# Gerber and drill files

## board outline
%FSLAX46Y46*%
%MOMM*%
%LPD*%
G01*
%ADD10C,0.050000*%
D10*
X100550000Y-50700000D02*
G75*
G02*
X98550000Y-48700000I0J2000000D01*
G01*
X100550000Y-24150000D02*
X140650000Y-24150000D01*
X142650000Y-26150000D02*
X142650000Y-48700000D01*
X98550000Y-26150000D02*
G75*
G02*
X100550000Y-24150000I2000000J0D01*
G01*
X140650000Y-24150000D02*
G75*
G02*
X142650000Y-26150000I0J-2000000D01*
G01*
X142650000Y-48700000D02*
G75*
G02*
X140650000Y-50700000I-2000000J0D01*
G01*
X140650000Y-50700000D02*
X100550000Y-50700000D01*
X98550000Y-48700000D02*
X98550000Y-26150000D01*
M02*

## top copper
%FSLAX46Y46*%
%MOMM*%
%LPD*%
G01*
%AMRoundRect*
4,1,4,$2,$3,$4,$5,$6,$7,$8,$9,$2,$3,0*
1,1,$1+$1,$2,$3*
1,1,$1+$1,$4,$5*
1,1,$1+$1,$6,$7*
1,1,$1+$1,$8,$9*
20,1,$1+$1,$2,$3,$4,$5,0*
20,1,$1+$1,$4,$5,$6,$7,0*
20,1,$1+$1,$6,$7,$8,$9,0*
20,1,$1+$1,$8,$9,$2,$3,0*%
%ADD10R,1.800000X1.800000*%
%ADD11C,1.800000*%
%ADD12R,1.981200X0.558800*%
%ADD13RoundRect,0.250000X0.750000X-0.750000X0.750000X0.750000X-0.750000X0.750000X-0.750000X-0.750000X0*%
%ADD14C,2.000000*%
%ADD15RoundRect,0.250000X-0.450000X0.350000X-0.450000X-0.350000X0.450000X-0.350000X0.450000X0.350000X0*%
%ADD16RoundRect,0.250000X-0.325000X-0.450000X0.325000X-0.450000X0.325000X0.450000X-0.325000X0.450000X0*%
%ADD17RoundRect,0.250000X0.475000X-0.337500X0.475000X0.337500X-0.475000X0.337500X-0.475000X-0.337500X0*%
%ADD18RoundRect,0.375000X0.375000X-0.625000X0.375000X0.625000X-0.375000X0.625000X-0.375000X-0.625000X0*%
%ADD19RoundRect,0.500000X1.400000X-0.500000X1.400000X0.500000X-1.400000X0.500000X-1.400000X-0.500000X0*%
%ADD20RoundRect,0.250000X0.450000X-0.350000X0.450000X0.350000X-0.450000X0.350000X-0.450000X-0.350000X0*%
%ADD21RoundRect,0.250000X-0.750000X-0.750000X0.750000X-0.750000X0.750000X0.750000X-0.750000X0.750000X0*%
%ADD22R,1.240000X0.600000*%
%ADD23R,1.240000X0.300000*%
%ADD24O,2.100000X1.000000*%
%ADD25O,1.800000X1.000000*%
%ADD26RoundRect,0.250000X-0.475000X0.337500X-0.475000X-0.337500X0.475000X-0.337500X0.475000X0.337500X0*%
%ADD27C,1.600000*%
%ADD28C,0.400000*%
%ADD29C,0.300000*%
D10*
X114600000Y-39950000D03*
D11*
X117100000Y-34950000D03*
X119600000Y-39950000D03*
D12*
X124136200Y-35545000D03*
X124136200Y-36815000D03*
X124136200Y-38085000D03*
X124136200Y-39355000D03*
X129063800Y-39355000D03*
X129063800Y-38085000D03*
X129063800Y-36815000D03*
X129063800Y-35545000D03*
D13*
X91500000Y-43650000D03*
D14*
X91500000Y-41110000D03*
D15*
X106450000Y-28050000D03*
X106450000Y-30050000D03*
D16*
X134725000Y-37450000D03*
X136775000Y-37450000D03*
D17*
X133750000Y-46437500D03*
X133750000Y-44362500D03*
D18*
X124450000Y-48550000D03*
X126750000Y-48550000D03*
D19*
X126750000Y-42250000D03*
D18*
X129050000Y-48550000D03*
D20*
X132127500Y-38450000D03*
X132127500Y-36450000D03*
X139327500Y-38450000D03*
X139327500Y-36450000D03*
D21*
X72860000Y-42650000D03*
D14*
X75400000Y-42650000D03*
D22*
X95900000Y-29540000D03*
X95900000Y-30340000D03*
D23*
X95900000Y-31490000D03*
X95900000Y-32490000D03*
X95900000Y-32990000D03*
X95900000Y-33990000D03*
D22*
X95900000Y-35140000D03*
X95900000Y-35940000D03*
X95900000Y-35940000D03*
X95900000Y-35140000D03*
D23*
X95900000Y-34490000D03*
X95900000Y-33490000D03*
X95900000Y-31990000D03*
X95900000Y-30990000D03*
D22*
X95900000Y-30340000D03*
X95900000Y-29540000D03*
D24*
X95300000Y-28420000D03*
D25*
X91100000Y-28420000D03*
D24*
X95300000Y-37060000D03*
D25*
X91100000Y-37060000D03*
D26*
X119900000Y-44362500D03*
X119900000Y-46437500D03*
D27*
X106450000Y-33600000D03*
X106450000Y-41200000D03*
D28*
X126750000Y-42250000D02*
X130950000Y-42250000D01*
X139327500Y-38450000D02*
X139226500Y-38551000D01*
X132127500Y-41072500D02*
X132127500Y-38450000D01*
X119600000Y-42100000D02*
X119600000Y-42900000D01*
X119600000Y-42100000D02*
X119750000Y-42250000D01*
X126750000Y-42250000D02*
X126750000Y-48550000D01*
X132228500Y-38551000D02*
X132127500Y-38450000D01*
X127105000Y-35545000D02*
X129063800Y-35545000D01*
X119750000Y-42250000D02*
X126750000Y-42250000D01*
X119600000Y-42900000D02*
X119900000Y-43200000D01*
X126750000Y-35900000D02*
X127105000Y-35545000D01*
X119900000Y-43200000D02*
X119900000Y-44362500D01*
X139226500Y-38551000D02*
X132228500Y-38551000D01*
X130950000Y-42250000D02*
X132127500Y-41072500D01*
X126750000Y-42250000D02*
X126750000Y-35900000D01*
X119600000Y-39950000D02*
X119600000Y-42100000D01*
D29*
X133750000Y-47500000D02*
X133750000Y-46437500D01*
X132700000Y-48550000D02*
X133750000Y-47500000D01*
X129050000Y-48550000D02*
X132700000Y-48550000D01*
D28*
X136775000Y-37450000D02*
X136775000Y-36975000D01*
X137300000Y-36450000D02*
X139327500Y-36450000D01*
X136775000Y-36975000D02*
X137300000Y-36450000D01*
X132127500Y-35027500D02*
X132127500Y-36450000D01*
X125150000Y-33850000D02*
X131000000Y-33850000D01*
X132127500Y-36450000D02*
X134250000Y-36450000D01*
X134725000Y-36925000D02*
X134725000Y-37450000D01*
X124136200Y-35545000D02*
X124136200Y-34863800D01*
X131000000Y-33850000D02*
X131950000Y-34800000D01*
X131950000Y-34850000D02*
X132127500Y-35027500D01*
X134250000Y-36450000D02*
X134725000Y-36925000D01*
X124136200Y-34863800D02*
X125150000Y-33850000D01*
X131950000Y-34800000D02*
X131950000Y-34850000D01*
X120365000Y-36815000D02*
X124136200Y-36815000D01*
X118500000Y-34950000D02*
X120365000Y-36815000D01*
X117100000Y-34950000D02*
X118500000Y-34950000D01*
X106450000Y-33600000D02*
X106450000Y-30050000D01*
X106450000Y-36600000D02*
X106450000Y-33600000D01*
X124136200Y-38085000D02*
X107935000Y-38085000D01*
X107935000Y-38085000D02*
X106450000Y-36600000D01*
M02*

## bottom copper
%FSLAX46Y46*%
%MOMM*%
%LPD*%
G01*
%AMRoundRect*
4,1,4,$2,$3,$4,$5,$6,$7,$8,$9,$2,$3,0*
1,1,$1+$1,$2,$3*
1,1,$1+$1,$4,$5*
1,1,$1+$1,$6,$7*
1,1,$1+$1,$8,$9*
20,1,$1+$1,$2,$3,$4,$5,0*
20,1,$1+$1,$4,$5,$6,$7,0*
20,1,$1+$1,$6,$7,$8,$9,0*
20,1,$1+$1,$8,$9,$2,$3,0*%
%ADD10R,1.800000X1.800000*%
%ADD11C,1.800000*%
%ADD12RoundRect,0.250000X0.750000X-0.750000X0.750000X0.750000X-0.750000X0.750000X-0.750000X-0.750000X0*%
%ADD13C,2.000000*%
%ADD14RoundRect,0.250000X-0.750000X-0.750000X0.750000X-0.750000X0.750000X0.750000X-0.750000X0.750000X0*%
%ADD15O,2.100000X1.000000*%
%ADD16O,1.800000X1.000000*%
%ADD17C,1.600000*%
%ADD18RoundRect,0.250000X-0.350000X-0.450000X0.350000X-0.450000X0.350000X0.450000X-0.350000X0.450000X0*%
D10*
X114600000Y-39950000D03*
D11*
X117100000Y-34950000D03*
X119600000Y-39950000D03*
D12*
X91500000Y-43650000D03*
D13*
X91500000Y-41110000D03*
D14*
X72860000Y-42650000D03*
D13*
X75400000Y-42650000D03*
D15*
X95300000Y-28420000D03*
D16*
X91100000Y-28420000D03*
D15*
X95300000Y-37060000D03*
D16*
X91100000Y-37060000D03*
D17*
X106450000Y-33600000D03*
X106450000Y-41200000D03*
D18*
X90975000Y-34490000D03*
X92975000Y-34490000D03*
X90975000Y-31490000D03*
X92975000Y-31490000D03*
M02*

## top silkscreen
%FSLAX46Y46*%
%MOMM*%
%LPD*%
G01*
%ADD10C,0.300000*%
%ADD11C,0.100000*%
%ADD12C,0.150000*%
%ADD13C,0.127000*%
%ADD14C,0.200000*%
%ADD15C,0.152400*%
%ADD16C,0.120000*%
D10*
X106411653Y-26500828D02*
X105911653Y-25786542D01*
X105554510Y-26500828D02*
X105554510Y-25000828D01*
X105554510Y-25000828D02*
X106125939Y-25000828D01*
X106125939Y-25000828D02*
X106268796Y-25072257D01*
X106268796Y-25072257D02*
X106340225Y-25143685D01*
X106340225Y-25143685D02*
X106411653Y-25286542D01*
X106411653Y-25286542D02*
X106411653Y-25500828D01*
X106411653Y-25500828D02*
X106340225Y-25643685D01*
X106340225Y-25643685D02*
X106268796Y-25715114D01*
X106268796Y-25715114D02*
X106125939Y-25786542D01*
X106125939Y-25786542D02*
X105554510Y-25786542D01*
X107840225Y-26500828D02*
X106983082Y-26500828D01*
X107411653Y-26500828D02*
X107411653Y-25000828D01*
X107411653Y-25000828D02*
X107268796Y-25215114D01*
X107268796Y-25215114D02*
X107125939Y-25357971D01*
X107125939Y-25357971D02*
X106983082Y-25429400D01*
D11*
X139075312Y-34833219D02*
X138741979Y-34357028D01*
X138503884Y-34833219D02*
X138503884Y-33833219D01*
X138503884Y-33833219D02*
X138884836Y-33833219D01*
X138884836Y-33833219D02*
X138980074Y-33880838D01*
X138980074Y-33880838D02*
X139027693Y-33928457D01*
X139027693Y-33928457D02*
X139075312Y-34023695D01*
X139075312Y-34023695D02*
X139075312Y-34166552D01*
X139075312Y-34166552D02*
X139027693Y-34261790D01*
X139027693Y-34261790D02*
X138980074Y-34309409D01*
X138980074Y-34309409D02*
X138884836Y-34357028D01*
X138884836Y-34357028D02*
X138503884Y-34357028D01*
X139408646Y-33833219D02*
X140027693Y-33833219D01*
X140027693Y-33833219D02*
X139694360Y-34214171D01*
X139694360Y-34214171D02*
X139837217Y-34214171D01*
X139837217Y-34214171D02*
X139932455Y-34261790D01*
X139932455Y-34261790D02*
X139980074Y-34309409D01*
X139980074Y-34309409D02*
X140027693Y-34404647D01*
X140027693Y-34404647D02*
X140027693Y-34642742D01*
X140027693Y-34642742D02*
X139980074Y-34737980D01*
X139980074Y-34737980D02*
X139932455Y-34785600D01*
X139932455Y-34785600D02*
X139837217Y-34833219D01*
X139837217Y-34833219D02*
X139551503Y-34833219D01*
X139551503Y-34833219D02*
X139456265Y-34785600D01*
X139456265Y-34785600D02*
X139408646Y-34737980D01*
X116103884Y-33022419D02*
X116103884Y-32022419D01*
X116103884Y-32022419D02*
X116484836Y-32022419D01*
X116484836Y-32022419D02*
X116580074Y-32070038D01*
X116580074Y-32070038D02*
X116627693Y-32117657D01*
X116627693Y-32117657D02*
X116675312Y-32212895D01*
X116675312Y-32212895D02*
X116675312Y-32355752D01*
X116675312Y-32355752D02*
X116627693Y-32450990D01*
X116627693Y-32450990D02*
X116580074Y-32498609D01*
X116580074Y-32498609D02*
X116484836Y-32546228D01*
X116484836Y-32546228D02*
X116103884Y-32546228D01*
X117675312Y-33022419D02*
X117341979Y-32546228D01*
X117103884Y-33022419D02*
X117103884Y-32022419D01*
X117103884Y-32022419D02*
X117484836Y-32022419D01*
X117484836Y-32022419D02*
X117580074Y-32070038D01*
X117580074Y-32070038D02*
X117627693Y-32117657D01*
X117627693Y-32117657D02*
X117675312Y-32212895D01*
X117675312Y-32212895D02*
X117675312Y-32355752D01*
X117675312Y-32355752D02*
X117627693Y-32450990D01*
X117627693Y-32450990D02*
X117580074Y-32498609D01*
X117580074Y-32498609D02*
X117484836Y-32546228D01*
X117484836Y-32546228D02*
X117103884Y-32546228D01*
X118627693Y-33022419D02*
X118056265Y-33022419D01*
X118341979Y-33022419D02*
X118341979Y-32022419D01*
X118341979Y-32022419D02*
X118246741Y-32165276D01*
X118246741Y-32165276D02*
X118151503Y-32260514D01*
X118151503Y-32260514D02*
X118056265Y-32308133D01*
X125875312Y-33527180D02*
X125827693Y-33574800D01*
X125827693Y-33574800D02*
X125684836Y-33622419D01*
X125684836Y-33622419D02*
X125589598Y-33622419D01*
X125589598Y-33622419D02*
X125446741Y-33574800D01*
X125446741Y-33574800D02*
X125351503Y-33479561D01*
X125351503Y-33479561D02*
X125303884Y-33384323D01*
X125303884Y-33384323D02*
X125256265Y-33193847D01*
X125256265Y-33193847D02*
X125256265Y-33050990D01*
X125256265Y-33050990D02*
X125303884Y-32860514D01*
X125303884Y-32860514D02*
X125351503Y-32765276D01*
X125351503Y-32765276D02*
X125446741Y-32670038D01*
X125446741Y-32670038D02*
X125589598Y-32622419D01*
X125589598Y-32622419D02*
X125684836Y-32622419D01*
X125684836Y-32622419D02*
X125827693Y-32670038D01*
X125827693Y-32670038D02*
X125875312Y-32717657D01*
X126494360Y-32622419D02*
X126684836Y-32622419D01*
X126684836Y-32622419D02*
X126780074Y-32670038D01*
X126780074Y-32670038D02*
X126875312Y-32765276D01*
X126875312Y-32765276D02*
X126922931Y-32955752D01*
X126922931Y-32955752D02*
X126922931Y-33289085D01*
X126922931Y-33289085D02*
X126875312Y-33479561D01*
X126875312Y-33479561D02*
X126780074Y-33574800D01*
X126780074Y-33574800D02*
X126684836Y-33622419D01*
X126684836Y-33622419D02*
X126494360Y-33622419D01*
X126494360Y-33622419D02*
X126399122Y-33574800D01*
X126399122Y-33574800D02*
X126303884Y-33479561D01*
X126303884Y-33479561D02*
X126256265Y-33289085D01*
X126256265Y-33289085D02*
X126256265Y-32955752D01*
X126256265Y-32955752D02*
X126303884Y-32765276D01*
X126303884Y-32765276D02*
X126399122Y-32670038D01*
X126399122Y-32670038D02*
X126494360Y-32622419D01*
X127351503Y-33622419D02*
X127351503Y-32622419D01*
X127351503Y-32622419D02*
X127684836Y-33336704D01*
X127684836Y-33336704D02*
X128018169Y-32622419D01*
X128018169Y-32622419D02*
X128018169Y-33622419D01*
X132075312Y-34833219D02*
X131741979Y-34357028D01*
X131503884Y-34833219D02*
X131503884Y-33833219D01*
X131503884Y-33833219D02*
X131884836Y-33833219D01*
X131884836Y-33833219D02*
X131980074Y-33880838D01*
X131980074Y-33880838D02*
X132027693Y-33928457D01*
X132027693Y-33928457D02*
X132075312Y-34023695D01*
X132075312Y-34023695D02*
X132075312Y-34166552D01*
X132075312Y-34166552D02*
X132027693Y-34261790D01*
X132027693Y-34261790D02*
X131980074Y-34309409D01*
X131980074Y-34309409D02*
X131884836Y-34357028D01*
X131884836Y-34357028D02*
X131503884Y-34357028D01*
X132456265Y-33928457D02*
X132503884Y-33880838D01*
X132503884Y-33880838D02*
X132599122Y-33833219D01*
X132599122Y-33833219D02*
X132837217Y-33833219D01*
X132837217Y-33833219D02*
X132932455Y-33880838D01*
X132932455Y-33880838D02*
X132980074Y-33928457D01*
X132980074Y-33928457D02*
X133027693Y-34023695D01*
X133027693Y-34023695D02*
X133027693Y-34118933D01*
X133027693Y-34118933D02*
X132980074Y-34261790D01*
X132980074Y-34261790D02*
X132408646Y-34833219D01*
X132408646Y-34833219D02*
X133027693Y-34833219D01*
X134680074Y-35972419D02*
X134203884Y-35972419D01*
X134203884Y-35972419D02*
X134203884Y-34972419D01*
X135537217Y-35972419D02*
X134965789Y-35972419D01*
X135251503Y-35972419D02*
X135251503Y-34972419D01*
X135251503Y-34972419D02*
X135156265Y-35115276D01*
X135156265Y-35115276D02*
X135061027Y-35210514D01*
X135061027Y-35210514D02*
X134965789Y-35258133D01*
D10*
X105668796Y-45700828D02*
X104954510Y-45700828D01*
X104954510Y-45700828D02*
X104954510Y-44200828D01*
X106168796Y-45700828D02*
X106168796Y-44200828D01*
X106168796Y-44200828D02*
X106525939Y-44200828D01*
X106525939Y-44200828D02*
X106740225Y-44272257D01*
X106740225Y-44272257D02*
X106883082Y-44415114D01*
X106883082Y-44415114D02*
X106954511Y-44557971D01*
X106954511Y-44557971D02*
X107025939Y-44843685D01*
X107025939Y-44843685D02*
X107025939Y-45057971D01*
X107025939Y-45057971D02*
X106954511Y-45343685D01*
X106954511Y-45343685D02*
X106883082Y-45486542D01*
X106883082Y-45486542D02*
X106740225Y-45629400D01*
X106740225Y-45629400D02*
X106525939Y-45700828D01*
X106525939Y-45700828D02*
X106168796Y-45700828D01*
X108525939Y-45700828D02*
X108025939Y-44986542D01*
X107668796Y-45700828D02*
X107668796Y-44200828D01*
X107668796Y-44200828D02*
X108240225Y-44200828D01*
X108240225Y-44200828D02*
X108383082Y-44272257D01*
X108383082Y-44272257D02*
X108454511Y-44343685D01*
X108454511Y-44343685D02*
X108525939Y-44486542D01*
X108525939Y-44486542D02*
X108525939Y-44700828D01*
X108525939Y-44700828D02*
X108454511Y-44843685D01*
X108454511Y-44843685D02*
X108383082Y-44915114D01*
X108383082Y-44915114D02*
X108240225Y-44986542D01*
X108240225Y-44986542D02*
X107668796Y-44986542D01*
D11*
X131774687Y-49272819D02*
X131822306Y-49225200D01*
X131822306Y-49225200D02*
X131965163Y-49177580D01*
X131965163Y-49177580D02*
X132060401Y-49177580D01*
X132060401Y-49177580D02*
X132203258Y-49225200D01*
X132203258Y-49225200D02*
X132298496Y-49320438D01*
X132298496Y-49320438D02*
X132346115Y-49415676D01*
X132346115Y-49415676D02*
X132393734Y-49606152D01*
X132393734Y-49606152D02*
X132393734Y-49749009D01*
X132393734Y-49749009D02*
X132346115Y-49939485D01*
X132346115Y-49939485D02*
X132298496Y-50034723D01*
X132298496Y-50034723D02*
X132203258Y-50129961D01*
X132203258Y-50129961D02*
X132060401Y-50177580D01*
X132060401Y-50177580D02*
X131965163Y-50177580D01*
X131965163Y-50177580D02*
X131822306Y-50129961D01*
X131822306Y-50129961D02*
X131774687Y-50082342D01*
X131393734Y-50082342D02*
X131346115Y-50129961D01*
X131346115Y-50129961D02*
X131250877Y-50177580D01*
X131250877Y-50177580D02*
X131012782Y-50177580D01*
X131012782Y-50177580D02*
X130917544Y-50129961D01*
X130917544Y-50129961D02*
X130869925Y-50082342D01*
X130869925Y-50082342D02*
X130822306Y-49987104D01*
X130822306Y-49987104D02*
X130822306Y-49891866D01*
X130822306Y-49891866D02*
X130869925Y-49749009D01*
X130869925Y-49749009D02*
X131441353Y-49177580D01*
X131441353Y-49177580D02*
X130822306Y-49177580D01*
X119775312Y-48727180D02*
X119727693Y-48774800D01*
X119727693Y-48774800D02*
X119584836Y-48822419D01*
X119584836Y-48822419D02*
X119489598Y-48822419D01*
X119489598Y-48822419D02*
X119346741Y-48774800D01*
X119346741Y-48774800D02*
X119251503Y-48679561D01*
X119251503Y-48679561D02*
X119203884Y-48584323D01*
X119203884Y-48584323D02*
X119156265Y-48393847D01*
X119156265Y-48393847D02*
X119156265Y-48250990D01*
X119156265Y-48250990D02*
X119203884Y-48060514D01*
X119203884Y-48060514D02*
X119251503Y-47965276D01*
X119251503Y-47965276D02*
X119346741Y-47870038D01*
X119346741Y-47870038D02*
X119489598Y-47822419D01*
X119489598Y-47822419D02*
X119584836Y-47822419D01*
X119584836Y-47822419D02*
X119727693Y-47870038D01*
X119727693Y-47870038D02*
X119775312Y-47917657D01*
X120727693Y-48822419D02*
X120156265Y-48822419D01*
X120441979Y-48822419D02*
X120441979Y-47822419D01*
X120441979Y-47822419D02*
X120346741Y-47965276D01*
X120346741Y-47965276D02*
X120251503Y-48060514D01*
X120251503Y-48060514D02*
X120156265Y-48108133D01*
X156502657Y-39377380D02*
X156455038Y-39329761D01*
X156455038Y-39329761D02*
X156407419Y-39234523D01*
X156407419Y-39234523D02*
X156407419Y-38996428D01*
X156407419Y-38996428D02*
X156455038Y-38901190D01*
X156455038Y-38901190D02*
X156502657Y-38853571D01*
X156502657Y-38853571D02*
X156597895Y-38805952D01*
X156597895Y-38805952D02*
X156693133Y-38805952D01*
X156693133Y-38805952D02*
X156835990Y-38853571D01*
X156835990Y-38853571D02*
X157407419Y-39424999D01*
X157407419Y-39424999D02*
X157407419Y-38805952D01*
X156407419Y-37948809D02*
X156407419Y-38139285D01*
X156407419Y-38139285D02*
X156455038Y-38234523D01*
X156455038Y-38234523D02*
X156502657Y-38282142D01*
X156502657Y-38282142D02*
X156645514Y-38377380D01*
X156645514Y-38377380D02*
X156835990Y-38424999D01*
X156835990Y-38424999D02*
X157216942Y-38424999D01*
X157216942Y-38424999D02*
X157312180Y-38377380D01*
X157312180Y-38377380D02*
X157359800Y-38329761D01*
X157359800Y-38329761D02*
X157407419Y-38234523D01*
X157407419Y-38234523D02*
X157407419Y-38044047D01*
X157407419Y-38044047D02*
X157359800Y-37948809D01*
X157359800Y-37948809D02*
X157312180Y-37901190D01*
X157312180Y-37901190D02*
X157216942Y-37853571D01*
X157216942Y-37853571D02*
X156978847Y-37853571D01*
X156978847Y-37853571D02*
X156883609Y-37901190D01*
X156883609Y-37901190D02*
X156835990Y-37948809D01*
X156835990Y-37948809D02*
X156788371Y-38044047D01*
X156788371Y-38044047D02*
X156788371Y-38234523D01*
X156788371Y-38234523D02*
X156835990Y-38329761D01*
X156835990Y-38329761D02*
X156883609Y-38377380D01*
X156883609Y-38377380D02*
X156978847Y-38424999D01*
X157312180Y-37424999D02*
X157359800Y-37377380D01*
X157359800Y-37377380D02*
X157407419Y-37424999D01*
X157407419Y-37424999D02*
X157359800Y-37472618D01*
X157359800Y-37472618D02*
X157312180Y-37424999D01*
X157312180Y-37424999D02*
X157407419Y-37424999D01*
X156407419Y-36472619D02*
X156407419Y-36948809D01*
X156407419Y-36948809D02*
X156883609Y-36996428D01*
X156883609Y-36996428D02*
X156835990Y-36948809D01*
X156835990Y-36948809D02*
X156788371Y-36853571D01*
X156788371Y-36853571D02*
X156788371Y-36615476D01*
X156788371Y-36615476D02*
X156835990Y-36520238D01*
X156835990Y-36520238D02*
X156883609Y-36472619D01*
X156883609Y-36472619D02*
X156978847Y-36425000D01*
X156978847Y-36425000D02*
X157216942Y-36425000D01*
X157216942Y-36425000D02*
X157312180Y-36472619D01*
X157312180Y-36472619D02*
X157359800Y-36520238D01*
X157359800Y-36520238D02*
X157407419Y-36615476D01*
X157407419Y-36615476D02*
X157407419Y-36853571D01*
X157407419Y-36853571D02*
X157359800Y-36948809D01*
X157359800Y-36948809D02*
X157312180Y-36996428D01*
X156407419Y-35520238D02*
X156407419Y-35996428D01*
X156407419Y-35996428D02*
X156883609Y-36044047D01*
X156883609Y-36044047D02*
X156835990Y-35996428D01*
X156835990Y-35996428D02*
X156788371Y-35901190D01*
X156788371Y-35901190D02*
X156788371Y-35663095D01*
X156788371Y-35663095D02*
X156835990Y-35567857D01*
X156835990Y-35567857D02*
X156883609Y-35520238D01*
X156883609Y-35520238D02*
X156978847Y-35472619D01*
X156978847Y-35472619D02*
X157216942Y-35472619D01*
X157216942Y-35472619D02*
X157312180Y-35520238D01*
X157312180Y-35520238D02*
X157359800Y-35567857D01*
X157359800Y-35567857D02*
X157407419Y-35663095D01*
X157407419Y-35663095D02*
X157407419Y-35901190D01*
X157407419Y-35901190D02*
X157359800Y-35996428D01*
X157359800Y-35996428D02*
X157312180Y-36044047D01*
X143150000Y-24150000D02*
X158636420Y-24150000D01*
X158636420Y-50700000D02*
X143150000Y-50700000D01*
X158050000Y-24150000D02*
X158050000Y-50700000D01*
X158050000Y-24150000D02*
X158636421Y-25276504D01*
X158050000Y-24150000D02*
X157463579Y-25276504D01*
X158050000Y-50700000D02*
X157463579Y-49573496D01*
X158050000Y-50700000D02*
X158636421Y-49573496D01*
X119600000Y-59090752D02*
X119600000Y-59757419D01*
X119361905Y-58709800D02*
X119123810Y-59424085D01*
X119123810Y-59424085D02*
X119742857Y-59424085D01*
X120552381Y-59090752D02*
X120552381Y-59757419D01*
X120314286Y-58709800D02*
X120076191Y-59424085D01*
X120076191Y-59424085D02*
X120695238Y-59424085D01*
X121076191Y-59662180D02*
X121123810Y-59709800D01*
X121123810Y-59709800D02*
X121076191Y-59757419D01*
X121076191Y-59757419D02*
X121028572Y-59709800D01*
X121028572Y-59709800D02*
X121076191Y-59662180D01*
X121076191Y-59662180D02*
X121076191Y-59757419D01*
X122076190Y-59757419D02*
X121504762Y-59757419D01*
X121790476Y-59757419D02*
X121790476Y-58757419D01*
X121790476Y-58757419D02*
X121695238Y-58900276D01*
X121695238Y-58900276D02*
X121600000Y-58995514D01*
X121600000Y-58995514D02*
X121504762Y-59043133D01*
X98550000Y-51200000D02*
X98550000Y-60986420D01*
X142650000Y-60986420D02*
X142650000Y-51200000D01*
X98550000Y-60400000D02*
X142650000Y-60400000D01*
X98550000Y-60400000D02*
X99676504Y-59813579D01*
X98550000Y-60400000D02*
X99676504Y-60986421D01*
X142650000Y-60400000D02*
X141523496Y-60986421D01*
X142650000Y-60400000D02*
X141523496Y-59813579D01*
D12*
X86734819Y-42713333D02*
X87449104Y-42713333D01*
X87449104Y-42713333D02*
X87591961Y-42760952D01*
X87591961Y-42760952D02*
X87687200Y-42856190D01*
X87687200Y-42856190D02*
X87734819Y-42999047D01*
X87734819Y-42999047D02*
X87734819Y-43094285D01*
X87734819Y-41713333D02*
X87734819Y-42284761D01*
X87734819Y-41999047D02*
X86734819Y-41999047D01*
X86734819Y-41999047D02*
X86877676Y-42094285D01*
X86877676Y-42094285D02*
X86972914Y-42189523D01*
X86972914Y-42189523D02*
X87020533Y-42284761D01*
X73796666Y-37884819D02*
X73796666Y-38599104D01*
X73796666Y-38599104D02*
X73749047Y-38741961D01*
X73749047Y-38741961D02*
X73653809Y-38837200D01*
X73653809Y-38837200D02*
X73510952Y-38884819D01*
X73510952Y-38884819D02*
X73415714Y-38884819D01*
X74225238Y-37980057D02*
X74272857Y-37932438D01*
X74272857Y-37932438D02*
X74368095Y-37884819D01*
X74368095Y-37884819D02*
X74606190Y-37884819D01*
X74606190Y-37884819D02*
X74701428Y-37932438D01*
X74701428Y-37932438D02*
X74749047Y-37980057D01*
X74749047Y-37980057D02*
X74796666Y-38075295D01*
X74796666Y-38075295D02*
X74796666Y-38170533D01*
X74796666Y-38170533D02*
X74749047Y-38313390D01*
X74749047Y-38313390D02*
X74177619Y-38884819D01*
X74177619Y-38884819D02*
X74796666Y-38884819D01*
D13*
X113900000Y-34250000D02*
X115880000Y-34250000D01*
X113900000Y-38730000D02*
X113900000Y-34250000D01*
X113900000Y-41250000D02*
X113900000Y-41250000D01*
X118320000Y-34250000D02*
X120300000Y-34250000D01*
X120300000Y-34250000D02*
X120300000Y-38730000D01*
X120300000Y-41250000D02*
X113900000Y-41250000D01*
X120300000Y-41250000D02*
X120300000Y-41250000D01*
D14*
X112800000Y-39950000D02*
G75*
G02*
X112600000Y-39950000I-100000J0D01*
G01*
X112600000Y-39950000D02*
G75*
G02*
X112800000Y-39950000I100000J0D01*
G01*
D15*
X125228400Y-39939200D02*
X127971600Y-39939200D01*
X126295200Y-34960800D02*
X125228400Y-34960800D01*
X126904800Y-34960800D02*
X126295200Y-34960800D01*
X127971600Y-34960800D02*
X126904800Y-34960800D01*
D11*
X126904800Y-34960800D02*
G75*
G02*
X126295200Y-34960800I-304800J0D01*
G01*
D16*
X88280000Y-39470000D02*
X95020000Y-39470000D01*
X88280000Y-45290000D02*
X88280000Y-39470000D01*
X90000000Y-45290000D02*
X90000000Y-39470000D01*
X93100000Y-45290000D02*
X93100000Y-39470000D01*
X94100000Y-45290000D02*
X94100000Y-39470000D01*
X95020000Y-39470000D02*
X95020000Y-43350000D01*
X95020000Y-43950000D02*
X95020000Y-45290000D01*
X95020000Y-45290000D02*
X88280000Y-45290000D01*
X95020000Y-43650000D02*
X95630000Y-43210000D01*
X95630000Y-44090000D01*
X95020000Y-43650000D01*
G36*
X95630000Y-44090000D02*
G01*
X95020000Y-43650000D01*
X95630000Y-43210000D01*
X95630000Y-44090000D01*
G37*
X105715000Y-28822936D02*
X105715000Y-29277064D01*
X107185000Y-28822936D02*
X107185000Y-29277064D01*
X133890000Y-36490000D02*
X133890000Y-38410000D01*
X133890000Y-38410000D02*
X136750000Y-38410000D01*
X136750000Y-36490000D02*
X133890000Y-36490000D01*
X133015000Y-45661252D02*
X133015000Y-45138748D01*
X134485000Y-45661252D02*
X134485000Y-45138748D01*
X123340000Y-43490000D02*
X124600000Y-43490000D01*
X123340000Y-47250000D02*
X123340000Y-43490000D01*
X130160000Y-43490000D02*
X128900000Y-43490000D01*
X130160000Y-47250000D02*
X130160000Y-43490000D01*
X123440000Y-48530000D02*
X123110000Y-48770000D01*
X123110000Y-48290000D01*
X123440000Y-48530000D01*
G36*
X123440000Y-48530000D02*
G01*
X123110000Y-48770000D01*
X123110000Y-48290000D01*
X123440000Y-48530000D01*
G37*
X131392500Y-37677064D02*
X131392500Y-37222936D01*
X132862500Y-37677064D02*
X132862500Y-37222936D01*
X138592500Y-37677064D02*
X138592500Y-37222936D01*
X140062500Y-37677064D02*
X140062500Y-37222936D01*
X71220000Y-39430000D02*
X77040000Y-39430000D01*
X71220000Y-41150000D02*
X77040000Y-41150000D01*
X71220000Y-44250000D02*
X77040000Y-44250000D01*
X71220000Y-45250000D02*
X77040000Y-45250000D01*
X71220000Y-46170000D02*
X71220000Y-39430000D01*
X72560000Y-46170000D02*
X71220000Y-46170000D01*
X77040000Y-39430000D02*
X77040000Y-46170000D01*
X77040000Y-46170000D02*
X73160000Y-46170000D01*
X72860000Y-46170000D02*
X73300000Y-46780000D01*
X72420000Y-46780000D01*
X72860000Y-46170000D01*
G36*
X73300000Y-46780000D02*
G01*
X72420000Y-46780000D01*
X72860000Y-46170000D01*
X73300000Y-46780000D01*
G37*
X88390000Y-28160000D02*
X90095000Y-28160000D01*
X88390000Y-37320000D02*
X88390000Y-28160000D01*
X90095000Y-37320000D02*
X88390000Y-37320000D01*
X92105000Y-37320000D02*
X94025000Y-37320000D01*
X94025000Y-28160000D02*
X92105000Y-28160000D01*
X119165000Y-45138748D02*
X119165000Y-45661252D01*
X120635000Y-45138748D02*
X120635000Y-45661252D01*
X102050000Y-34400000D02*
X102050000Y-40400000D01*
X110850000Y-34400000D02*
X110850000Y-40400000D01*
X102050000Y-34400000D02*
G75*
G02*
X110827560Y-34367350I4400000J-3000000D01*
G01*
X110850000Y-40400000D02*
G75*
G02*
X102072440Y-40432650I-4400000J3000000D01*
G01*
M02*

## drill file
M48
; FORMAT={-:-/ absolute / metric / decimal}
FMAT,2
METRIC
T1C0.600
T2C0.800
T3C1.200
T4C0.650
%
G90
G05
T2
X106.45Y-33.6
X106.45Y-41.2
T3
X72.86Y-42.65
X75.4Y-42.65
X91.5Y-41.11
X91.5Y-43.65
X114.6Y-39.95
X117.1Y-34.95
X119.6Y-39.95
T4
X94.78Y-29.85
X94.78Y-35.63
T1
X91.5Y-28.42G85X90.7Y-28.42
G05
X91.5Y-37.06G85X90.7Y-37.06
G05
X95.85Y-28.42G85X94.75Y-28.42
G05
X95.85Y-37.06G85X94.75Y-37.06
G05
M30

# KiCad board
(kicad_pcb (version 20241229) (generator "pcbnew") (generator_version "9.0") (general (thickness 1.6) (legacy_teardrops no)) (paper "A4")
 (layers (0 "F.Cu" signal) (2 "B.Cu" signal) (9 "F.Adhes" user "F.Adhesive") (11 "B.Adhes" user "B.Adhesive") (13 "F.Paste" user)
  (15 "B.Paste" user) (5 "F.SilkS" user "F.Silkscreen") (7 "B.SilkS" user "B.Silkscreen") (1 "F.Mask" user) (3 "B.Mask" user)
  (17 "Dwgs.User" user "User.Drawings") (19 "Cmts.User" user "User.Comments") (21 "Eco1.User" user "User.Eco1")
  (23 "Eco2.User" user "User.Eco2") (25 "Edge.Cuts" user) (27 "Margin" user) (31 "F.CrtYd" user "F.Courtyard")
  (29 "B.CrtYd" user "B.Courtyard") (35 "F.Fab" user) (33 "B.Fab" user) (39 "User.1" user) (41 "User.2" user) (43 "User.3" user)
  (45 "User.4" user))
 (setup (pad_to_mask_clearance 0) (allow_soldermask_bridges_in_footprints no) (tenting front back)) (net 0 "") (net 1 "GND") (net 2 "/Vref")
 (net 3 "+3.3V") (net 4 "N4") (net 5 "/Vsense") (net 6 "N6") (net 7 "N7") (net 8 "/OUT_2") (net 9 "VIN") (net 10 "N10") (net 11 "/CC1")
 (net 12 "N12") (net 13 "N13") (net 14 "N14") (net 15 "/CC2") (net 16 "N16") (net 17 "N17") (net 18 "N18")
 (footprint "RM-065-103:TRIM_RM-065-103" (layer "F.Cu") (at 117.1 37.45)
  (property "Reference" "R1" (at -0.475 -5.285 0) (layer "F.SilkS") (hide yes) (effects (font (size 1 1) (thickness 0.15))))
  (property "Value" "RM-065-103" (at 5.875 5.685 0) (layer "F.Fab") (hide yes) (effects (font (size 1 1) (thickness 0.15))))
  (fp_line (start -3.2 -3.2) (end -1.22 -3.2) (stroke (width 0.127) (type solid)) (layer "F.SilkS"))
  (fp_line (start -3.2 1.28) (end -3.2 -3.2) (stroke (width 0.127) (type solid)) (layer "F.SilkS"))
  (fp_line (start -3.2 3.8) (end -3.2 3.8) (stroke (width 0.127) (type solid)) (layer "F.SilkS"))
  (fp_line (start 1.22 -3.2) (end 3.2 -3.2) (stroke (width 0.127) (type solid)) (layer "F.SilkS"))
  (fp_line (start 3.2 -3.2) (end 3.2 1.28) (stroke (width 0.127) (type solid)) (layer "F.SilkS"))
  (fp_line (start 3.2 3.8) (end -3.2 3.8) (stroke (width 0.127) (type solid)) (layer "F.SilkS"))
  (fp_line (start 3.2 3.8) (end 3.2 3.8) (stroke (width 0.127) (type solid)) (layer "F.SilkS"))
  (fp_circle (center -4.4 2.5) (end -4.3 2.5) (stroke (width 0.2) (type solid)) (fill no) (layer "F.SilkS"))
  (pad "1" thru_hole rect (at -2.5 2.5) (size 1.8 1.8) (drill 1.2) (layers "*.Cu" "*.Mask") (remove_unused_layers no) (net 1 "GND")
   (solder_mask_margin 0.102))
  (pad "2" thru_hole circle (at 0 -2.5) (size 1.8 1.8) (drill 1.2) (layers "*.Cu" "*.Mask") (remove_unused_layers no) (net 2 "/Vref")
   (solder_mask_margin 0.102))
  (pad "3" thru_hole circle (at 2.5 2.5) (size 1.8 1.8) (drill 1.2) (layers "*.Cu" "*.Mask") (remove_unused_layers no) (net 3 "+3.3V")
   (solder_mask_margin 0.102)))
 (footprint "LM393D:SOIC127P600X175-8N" (layer "F.Cu") (at 126.6 37.45)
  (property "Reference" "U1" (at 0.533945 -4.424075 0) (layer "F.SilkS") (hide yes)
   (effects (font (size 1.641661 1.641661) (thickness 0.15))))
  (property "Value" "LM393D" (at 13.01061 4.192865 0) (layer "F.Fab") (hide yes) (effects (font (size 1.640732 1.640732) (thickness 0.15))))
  (fp_line (start -1.3716 2.4892) (end 1.3716 2.4892) (stroke (width 0.1524) (type solid)) (layer "F.SilkS"))
  (fp_line (start -0.3048 -2.4892) (end -1.3716 -2.4892) (stroke (width 0.1524) (type solid)) (layer "F.SilkS"))
  (fp_line (start 0.3048 -2.4892) (end -0.3048 -2.4892) (stroke (width 0.1524) (type solid)) (layer "F.SilkS"))
  (fp_line (start 1.3716 -2.4892) (end 0.3048 -2.4892) (stroke (width 0.1524) (type solid)) (layer "F.SilkS"))
  (fp_arc (start 0.3048 -2.4892) (mid 0 -2.1844) (end -0.3048 -2.4892) (stroke (width 0.1) (type solid)) (layer "F.SilkS"))
  (pad "1" smd rect (at -2.4638 -1.905) (size 1.9812 0.5588) (layers "F.Cu" "F.Mask" "F.Paste") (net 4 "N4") (solder_mask_margin 0.102))
  (pad "2" smd rect (at -2.4638 -0.635) (size 1.9812 0.5588) (layers "F.Cu" "F.Mask" "F.Paste") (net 2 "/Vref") (solder_mask_margin 0.102))
  (pad "3" smd rect (at -2.4638 0.635) (size 1.9812 0.5588) (layers "F.Cu" "F.Mask" "F.Paste") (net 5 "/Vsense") (solder_mask_margin 0.102))
  (pad "4" smd rect (at -2.4638 1.905) (size 1.9812 0.5588) (layers "F.Cu" "F.Mask" "F.Paste") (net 1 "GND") (solder_mask_margin 0.102))
  (pad "5" smd rect (at 2.4638 1.905) (size 1.9812 0.5588) (layers "F.Cu" "F.Mask" "F.Paste") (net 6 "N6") (solder_mask_margin 0.102))
  (pad "6" smd rect (at 2.4638 0.635) (size 1.9812 0.5588) (layers "F.Cu" "F.Mask" "F.Paste") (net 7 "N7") (solder_mask_margin 0.102))
  (pad "7" smd rect (at 2.4638 -0.635) (size 1.9812 0.5588) (layers "F.Cu" "F.Mask" "F.Paste") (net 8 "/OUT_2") (solder_mask_margin 0.102))
  (pad "8" smd rect (at 2.4638 -1.905) (size 1.9812 0.5588) (layers "F.Cu" "F.Mask" "F.Paste") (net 3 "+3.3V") (solder_mask_margin 0.102)))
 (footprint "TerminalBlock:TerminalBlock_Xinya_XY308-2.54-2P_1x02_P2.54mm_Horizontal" (layer "F.Cu") (at 91.5 43.65 90)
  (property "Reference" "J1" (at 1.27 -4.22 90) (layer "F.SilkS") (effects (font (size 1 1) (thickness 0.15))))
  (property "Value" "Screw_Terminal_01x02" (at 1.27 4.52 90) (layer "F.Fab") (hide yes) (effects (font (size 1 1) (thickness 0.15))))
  (fp_line (start 4.18 -3.22) (end 4.18 3.52) (stroke (width 0.12) (type solid)) (layer "F.SilkS"))
  (fp_line (start -1.64 -3.22) (end 4.18 -3.22) (stroke (width 0.12) (type solid)) (layer "F.SilkS"))
  (fp_line (start -1.64 -1.5) (end 4.18 -1.5) (stroke (width 0.12) (type solid)) (layer "F.SilkS"))
  (fp_line (start -1.64 1.6) (end 4.18 1.6) (stroke (width 0.12) (type solid)) (layer "F.SilkS"))
  (fp_line (start -1.64 2.6) (end 4.18 2.6) (stroke (width 0.12) (type solid)) (layer "F.SilkS"))
  (fp_line (start 4.18 3.52) (end 0.3 3.52) (stroke (width 0.12) (type solid)) (layer "F.SilkS"))
  (fp_line (start -0.3 3.52) (end -1.64 3.52) (stroke (width 0.12) (type solid)) (layer "F.SilkS"))
  (fp_line (start -1.64 3.52) (end -1.64 -3.22) (stroke (width 0.12) (type solid)) (layer "F.SilkS"))
  (fp_poly (pts (xy 0 3.52) (xy 0.44 4.13) (xy -0.44 4.13)) (stroke (width 0.12) (type solid)) (fill yes) (layer "F.SilkS"))
  (pad "1" thru_hole roundrect (at 0 0 90) (size 2 2) (drill 1.2) (layers "*.Cu" "*.Mask") (remove_unused_layers no)
   (roundrect_rratio 0.125) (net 1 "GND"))
  (pad "2" thru_hole circle (at 2.54 0 90) (size 2 2) (drill 1.2) (layers "*.Cu" "*.Mask") (remove_unused_layers no) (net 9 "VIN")))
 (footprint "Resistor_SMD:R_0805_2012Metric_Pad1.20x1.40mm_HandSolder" (layer "F.Cu") (at 106.45 29.05 -90)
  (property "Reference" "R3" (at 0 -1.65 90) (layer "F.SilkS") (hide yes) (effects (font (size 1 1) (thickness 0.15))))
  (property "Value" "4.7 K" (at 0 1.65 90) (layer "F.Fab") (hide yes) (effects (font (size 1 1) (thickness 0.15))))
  (fp_line (start -0.227064 0.735) (end 0.227064 0.735) (stroke (width 0.12) (type solid)) (layer "F.SilkS"))
  (fp_line (start -0.227064 -0.735) (end 0.227064 -0.735) (stroke (width 0.12) (type solid)) (layer "F.SilkS"))
  (pad "1" smd roundrect (at -1 0 270) (size 1.2 1.4) (layers "F.Cu" "F.Mask" "F.Paste") (roundrect_rratio 0.208333) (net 3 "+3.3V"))
  (pad "2" smd roundrect (at 1 0 270) (size 1.2 1.4) (layers "F.Cu" "F.Mask" "F.Paste") (roundrect_rratio 0.208333) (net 5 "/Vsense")))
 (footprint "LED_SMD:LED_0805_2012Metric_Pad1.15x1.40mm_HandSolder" (layer "F.Cu") (at 135.75 37.45)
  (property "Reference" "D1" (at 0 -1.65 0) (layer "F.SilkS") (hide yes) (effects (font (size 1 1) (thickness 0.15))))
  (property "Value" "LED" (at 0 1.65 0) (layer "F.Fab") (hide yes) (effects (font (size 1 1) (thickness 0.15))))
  (fp_line (start -1.86 -0.96) (end -1.86 0.96) (stroke (width 0.12) (type solid)) (layer "F.SilkS"))
  (fp_line (start -1.86 0.96) (end 1 0.96) (stroke (width 0.12) (type solid)) (layer "F.SilkS"))
  (fp_line (start 1 -0.96) (end -1.86 -0.96) (stroke (width 0.12) (type solid)) (layer "F.SilkS"))
  (pad "1" smd roundrect (at -1.025 0) (size 1.15 1.4) (layers "F.Cu" "F.Mask" "F.Paste") (roundrect_rratio 0.217391) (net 4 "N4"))
  (pad "2" smd roundrect (at 1.025 0) (size 1.15 1.4) (layers "F.Cu" "F.Mask" "F.Paste") (roundrect_rratio 0.217391) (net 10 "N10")))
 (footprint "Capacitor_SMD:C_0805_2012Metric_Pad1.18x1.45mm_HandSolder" (layer "F.Cu") (at 133.75 45.4 90)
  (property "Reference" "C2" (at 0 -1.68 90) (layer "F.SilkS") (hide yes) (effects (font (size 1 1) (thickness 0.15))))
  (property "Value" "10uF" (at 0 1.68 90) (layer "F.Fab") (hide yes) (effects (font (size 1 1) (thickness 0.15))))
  (fp_line (start -0.261252 -0.735) (end 0.261252 -0.735) (stroke (width 0.12) (type solid)) (layer "F.SilkS"))
  (fp_line (start -0.261252 0.735) (end 0.261252 0.735) (stroke (width 0.12) (type solid)) (layer "F.SilkS"))
  (pad "1" smd roundrect (at -1.0375 0 90) (size 1.175 1.45) (layers "F.Cu" "F.Mask" "F.Paste") (roundrect_rratio 0.212766) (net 9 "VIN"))
  (pad "2" smd roundrect (at 1.0375 0 90) (size 1.175 1.45) (layers "F.Cu" "F.Mask" "F.Paste") (roundrect_rratio 0.212766) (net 1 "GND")))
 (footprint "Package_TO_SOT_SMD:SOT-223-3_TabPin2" (layer "F.Cu") (at 126.75 45.4 90)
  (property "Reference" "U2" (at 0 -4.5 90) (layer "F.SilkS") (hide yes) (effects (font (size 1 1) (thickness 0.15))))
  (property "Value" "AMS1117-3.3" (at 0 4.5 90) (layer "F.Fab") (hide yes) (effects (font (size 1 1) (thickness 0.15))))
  (fp_line (start 1.91 -3.41) (end 1.91 -2.15) (stroke (width 0.12) (type solid)) (layer "F.SilkS"))
  (fp_line (start -1.85 -3.41) (end 1.91 -3.41) (stroke (width 0.12) (type solid)) (layer "F.SilkS"))
  (fp_line (start 1.91 3.41) (end 1.91 2.15) (stroke (width 0.12) (type solid)) (layer "F.SilkS"))
  (fp_line (start -1.85 3.41) (end 1.91 3.41) (stroke (width 0.12) (type solid)) (layer "F.SilkS"))
  (fp_poly
   (pts (xy -3.13 -3.31) (xy -3.37 -3.64) (xy -2.89 -3.64) (xy -3.13 -3.31)) (stroke (width 0.12) (type solid)) (fill yes) (layer "F.SilkS"))
  (pad "1" smd roundrect (at -3.15 -2.3 90) (size 2 1.5) (layers "F.Cu" "F.Mask" "F.Paste") (roundrect_rratio 0.25) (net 1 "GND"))
  (pad "2" smd roundrect (at -3.15 0 90) (size 2 1.5) (layers "F.Cu" "F.Mask" "F.Paste") (roundrect_rratio 0.25) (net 3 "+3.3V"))
  (pad "2" smd roundrect (at 3.15 0 90) (size 2 3.8) (layers "F.Cu" "F.Mask" "F.Paste") (roundrect_rratio 0.25) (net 3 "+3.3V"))
  (pad "3" smd roundrect (at -3.15 2.3 90) (size 2 1.5) (layers "F.Cu" "F.Mask" "F.Paste") (roundrect_rratio 0.25) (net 9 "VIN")))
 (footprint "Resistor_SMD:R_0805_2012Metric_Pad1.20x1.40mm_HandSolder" (layer "F.Cu") (at 132.1275 37.45 90)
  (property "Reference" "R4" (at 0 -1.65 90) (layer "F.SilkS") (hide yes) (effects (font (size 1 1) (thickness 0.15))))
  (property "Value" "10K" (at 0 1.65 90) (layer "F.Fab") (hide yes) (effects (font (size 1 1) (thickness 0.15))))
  (fp_line (start -0.227064 -0.735) (end 0.227064 -0.735) (stroke (width 0.12) (type solid)) (layer "F.SilkS"))
  (fp_line (start -0.227064 0.735) (end 0.227064 0.735) (stroke (width 0.12) (type solid)) (layer "F.SilkS"))
  (pad "1" smd roundrect (at -1 0 90) (size 1.2 1.4) (layers "F.Cu" "F.Mask" "F.Paste") (roundrect_rratio 0.208333) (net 3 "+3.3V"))
  (pad "2" smd roundrect (at 1 0 90) (size 1.2 1.4) (layers "F.Cu" "F.Mask" "F.Paste") (roundrect_rratio 0.208333) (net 4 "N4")))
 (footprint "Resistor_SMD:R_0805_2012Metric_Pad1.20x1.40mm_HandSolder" (layer "F.Cu") (at 139.3275 37.45 90)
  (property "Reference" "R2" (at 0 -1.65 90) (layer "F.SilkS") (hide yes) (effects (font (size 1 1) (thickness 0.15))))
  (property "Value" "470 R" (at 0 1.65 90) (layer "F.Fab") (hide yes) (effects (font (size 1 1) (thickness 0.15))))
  (fp_line (start -0.227064 -0.735) (end 0.227064 -0.735) (stroke (width 0.12) (type solid)) (layer "F.SilkS"))
  (fp_line (start -0.227064 0.735) (end 0.227064 0.735) (stroke (width 0.12) (type solid)) (layer "F.SilkS"))
  (pad "1" smd roundrect (at -1 0 90) (size 1.2 1.4) (layers "F.Cu" "F.Mask" "F.Paste") (roundrect_rratio 0.208333) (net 3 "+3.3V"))
  (pad "2" smd roundrect (at 1 0 90) (size 1.2 1.4) (layers "F.Cu" "F.Mask" "F.Paste") (roundrect_rratio 0.208333) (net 10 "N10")))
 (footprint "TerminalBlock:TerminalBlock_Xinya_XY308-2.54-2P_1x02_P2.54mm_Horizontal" (layer "F.Cu") (at 72.86 42.65)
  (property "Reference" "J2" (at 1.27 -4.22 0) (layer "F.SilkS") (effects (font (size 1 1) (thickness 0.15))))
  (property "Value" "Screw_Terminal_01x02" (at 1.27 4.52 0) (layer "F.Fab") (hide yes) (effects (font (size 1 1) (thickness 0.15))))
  (fp_line (start -1.64 -3.22) (end 4.18 -3.22) (stroke (width 0.12) (type solid)) (layer "F.SilkS"))
  (fp_line (start -1.64 -1.5) (end 4.18 -1.5) (stroke (width 0.12) (type solid)) (layer "F.SilkS"))
  (fp_line (start -1.64 1.6) (end 4.18 1.6) (stroke (width 0.12) (type solid)) (layer "F.SilkS"))
  (fp_line (start -1.64 2.6) (end 4.18 2.6) (stroke (width 0.12) (type solid)) (layer "F.SilkS"))
  (fp_line (start -1.64 3.52) (end -1.64 -3.22) (stroke (width 0.12) (type solid)) (layer "F.SilkS"))
  (fp_line (start -0.3 3.52) (end -1.64 3.52) (stroke (width 0.12) (type solid)) (layer "F.SilkS"))
  (fp_line (start 4.18 -3.22) (end 4.18 3.52) (stroke (width 0.12) (type solid)) (layer "F.SilkS"))
  (fp_line (start 4.18 3.52) (end 0.3 3.52) (stroke (width 0.12) (type solid)) (layer "F.SilkS"))
  (fp_poly (pts (xy 0 3.52) (xy 0.44 4.13) (xy -0.44 4.13)) (stroke (width 0.12) (type solid)) (fill yes) (layer "F.SilkS"))
  (pad "1" thru_hole roundrect (at 0 0) (size 2 2) (drill 1.2) (layers "*.Cu" "*.Mask") (remove_unused_layers no) (roundrect_rratio 0.125)
   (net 1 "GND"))
  (pad "2" thru_hole circle (at 2.54 0) (size 2 2) (drill 1.2) (layers "*.Cu" "*.Mask") (remove_unused_layers no) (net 8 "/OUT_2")))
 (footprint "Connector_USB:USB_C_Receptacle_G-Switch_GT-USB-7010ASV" (layer "F.Cu") (at 92.175 32.74 -90)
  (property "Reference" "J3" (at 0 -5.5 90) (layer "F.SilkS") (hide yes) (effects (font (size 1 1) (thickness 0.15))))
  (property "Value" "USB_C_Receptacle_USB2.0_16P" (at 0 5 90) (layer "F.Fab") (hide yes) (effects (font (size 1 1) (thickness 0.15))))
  (fp_line (start -4.58 3.785) (end -4.58 2.08) (stroke (width 0.12) (type solid)) (layer "F.SilkS"))
  (fp_line (start 4.58 3.785) (end -4.58 3.785) (stroke (width 0.12) (type solid)) (layer "F.SilkS"))
  (fp_line (start 4.58 2.08) (end 4.58 3.785) (stroke (width 0.12) (type solid)) (layer "F.SilkS"))
  (fp_line (start 4.58 0.07) (end 4.58 -1.85) (stroke (width 0.12) (type solid)) (layer "F.SilkS"))
  (fp_line (start -4.58 -1.85) (end -4.58 0.07) (stroke (width 0.12) (type solid)) (layer "F.SilkS"))
  (pad "" np_thru_hole circle (at -2.89 -2.605 270) (size 0.65 0.65) (drill 0.65) (layers "*.Cu" "*.Mask"))
  (pad "" np_thru_hole circle (at 2.89 -2.605 270) (size 0.65 0.65) (drill 0.65) (layers "*.Cu" "*.Mask"))
  (pad "A1" smd rect (at -3.2 -3.725 270) (size 0.6 1.24) (layers "F.Cu" "F.Mask" "F.Paste") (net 1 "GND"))
  (pad "A4" smd rect (at -2.4 -3.725 270) (size 0.6 1.24) (layers "F.Cu" "F.Mask" "F.Paste") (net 9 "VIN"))
  (pad "A5" smd rect (at -1.25 -3.725 270) (size 0.3 1.24) (layers "F.Cu" "F.Mask" "F.Paste") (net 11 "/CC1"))
  (pad "A6" smd rect (at -0.25 -3.725 270) (size 0.3 1.24) (layers "F.Cu" "F.Mask" "F.Paste") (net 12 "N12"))
  (pad "A7" smd rect (at 0.25 -3.725 270) (size 0.3 1.24) (layers "F.Cu" "F.Mask" "F.Paste") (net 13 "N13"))
  (pad "A8" smd rect (at 1.25 -3.725 270) (size 0.3 1.24) (layers "F.Cu" "F.Mask" "F.Paste") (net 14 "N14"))
  (pad "A9" smd rect (at 2.4 -3.725 270) (size 0.6 1.24) (layers "F.Cu" "F.Mask" "F.Paste") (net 9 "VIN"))
  (pad "A12" smd rect (at 3.2 -3.725 270) (size 0.6 1.24) (layers "F.Cu" "F.Mask" "F.Paste") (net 1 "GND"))
  (pad "B1" smd rect (at 3.2 -3.725 270) (size 0.6 1.24) (layers "F.Cu" "F.Mask" "F.Paste") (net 1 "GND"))
  (pad "B4" smd rect (at 2.4 -3.725 270) (size 0.6 1.24) (layers "F.Cu" "F.Mask" "F.Paste") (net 9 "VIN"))
  (pad "B5" smd rect (at 1.75 -3.725 270) (size 0.3 1.24) (layers "F.Cu" "F.Mask" "F.Paste") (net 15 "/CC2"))
  (pad "B6" smd rect (at 0.75 -3.725 270) (size 0.3 1.24) (layers "F.Cu" "F.Mask" "F.Paste") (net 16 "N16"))
  (pad "B7" smd rect (at -0.75 -3.725 270) (size 0.3 1.24) (layers "F.Cu" "F.Mask" "F.Paste") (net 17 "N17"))
  (pad "B8" smd rect (at -1.75 -3.725 270) (size 0.3 1.24) (layers "F.Cu" "F.Mask" "F.Paste") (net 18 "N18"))
  (pad "B9" smd rect (at -2.4 -3.725 270) (size 0.6 1.24) (layers "F.Cu" "F.Mask" "F.Paste") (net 9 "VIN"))
  (pad "B12" smd rect (at -3.2 -3.725 270) (size 0.6 1.24) (layers "F.Cu" "F.Mask" "F.Paste") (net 1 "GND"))
  (pad "S1" thru_hole oval (at -4.32 -3.125 270) (size 1 2.1) (drill oval 0.6 1.7) (layers "*.Cu" "*.Mask") (remove_unused_layers no)
   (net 1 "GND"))
  (pad "S1" thru_hole oval (at -4.32 1.075 270) (size 1 1.8) (drill oval 0.6 1.4) (layers "*.Cu" "*.Mask") (remove_unused_layers no)
   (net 1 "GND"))
  (pad "S1" thru_hole oval (at 4.32 -3.125 270) (size 1 2.1) (drill oval 0.6 1.7) (layers "*.Cu" "*.Mask") (remove_unused_layers no)
   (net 1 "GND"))
  (pad "S1" thru_hole oval (at 4.32 1.075 270) (size 1 1.8) (drill oval 0.6 1.4) (layers "*.Cu" "*.Mask") (remove_unused_layers no)
   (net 1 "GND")))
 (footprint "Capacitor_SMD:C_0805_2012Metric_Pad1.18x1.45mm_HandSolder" (layer "F.Cu") (at 119.9 45.4 -90)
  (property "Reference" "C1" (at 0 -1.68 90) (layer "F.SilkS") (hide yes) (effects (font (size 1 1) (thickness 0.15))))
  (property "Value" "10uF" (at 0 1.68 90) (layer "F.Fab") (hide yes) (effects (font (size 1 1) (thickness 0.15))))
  (fp_line (start -0.261252 0.735) (end 0.261252 0.735) (stroke (width 0.12) (type solid)) (layer "F.SilkS"))
  (fp_line (start -0.261252 -0.735) (end 0.261252 -0.735) (stroke (width 0.12) (type solid)) (layer "F.SilkS"))
  (pad "1" smd roundrect (at -1.0375 0 270) (size 1.175 1.45) (layers "F.Cu" "F.Mask" "F.Paste") (roundrect_rratio 0.212766) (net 3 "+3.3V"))
  (pad "2" smd roundrect (at 1.0375 0 270) (size 1.175 1.45) (layers "F.Cu" "F.Mask" "F.Paste") (roundrect_rratio 0.212766) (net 1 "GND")))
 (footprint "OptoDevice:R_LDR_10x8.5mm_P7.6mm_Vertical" (layer "F.Cu") (at 106.45 33.6 -90)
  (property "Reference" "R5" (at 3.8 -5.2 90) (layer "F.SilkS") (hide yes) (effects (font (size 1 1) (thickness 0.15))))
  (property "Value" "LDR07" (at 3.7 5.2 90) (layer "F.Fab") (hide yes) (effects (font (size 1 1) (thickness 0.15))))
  (fp_line (start 0.8 4.4) (end 6.8 4.4) (stroke (width 0.12) (type solid)) (layer "F.SilkS"))
  (fp_line (start 0.8 -4.4) (end 6.8 -4.4) (stroke (width 0.12) (type solid)) (layer "F.SilkS"))
  (fp_arc (start 0.8 4.4) (mid -1.525374 0.019809) (end 0.76735 -4.37756) (stroke (width 0.12) (type solid)) (layer "F.SilkS"))
  (fp_arc (start 6.8 -4.4) (mid 9.125374 -0.019809) (end 6.83265 4.37756) (stroke (width 0.12) (type solid)) (layer "F.SilkS"))
  (pad "1" thru_hole circle (at 0 0 270) (size 1.6 1.6) (drill 0.8) (layers "*.Cu" "*.Mask") (remove_unused_layers no) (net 5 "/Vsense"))
  (pad "2" thru_hole circle (at 7.6 0 270) (size 1.6 1.6) (drill 0.8) (layers "*.Cu" "*.Mask") (remove_unused_layers no) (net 1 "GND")))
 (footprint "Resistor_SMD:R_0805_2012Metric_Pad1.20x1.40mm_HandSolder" (layer "B.Cu") (at 91.975 34.49)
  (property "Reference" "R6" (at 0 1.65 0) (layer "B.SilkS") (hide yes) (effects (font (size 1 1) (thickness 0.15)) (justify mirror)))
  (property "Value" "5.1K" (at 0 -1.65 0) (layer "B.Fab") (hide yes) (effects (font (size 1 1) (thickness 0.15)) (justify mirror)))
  (pad "1" smd roundrect (at -1 0) (size 1.2 1.4) (layers "B.Cu" "B.Mask" "B.Paste") (roundrect_rratio 0.208333) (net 1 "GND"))
  (pad "2" smd roundrect (at 1 0) (size 1.2 1.4) (layers "B.Cu" "B.Mask" "B.Paste") (roundrect_rratio 0.208333) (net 15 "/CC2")))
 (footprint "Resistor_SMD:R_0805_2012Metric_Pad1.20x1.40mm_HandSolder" (layer "B.Cu") (at 91.975 31.49)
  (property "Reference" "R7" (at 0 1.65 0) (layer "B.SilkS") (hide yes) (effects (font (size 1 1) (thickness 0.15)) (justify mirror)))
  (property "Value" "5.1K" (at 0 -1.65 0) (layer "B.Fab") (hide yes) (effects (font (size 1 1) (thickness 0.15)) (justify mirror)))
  (pad "1" smd roundrect (at -1 0) (size 1.2 1.4) (layers "B.Cu" "B.Mask" "B.Paste") (roundrect_rratio 0.208333) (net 1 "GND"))
  (pad "2" smd roundrect (at 1 0) (size 1.2 1.4) (layers "B.Cu" "B.Mask" "B.Paste") (roundrect_rratio 0.208333) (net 11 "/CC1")))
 (gr_arc (start 100.55 50.7) (mid 99.135786 50.114214) (end 98.55 48.7) (stroke (width 0.05) (type default)) (layer "Edge.Cuts"))
 (gr_line (start 100.55 24.15) (end 140.65 24.15) (stroke (width 0.05) (type default)) (layer "Edge.Cuts"))
 (gr_line (start 142.65 26.15) (end 142.65 48.7) (stroke (width 0.05) (type default)) (layer "Edge.Cuts"))
 (gr_arc (start 98.55 26.15) (mid 99.135786 24.735786) (end 100.55 24.15) (stroke (width 0.05) (type default)) (layer "Edge.Cuts"))
 (gr_arc (start 140.65 24.15) (mid 142.064214 24.735786) (end 142.65 26.15) (stroke (width 0.05) (type default)) (layer "Edge.Cuts"))
 (gr_arc (start 142.65 48.7) (mid 142.064214 50.114214) (end 140.65 50.7) (stroke (width 0.05) (type default)) (layer "Edge.Cuts"))
 (gr_line (start 140.65 50.7) (end 100.55 50.7) (stroke (width 0.05) (type default)) (layer "Edge.Cuts"))
 (gr_line (start 98.55 48.7) (end 98.55 26.15) (stroke (width 0.05) (type default)) (layer "Edge.Cuts"))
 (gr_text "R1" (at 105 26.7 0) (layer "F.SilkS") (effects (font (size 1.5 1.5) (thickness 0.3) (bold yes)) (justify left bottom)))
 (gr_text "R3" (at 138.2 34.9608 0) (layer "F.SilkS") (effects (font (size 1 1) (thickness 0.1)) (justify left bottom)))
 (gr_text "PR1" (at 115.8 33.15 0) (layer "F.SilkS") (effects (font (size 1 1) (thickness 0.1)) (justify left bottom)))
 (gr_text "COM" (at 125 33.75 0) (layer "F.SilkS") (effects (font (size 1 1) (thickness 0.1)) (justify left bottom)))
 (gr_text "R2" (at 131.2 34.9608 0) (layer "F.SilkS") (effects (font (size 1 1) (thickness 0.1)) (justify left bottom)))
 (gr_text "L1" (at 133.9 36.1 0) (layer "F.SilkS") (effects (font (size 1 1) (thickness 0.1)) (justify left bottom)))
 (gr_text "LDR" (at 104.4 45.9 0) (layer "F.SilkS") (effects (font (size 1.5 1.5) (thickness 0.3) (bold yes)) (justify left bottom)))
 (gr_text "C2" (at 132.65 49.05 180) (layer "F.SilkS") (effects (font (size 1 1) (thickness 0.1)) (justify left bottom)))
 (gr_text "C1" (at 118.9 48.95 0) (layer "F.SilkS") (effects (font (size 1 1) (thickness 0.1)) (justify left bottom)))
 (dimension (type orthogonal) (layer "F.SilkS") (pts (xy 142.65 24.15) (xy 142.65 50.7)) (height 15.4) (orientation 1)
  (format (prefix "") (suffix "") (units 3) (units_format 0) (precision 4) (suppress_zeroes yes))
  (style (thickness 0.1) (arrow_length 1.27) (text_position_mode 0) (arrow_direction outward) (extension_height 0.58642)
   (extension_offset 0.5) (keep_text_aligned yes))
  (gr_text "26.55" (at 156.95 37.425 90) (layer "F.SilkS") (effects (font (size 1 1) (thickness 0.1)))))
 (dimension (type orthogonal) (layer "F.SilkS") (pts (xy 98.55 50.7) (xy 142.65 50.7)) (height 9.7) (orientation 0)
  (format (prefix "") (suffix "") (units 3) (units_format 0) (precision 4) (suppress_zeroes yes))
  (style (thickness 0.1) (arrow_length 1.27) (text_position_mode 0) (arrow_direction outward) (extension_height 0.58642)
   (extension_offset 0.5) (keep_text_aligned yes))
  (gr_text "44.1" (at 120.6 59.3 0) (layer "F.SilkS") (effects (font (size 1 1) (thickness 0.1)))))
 (segment (start 126.75 42.25) (end 130.95 42.25) (width 0.4) (layer "F.Cu") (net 3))
 (segment (start 139.3275 38.45) (end 139.2265 38.551) (width 0.4) (layer "F.Cu") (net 3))
 (segment (start 132.1275 41.0725) (end 132.1275 38.45) (width 0.4) (layer "F.Cu") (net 3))
 (segment (start 119.6 42.1) (end 119.6 42.9) (width 0.4) (layer "F.Cu") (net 3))
 (segment (start 119.6 42.1) (end 119.75 42.25) (width 0.4) (layer "F.Cu") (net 3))
 (segment (start 126.75 42.25) (end 126.75 48.55) (width 0.4) (layer "F.Cu") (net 3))
 (segment (start 132.2285 38.551) (end 132.1275 38.45) (width 0.4) (layer "F.Cu") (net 3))
 (segment (start 127.105 35.545) (end 129.0638 35.545) (width 0.4) (layer "F.Cu") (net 3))
 (segment (start 119.75 42.25) (end 126.75 42.25) (width 0.4) (layer "F.Cu") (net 3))
 (segment (start 119.6 42.9) (end 119.9 43.2) (width 0.4) (layer "F.Cu") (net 3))
 (segment (start 126.75 35.9) (end 127.105 35.545) (width 0.4) (layer "F.Cu") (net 3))
 (segment (start 119.9 43.2) (end 119.9 44.3625) (width 0.4) (layer "F.Cu") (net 3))
 (segment (start 139.2265 38.551) (end 132.2285 38.551) (width 0.4) (layer "F.Cu") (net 3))
 (segment (start 130.95 42.25) (end 132.1275 41.0725) (width 0.4) (layer "F.Cu") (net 3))
 (segment (start 126.75 42.25) (end 126.75 35.9) (width 0.4) (layer "F.Cu") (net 3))
 (segment (start 119.6 39.95) (end 119.6 42.1) (width 0.4) (layer "F.Cu") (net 3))
 (segment (start 133.75 47.5) (end 133.75 46.4375) (width 0.3) (layer "F.Cu") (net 9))
 (segment (start 132.7 48.55) (end 133.75 47.5) (width 0.3) (layer "F.Cu") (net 9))
 (segment (start 129.05 48.55) (end 132.7 48.55) (width 0.3) (layer "F.Cu") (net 9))
 (segment (start 136.775 37.45) (end 136.775 36.975) (width 0.4) (layer "F.Cu") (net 10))
 (segment (start 137.3 36.45) (end 139.3275 36.45) (width 0.4) (layer "F.Cu") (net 10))
 (segment (start 136.775 36.975) (end 137.3 36.45) (width 0.4) (layer "F.Cu") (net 10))
 (segment (start 132.1275 35.0275) (end 132.1275 36.45) (width 0.4) (layer "F.Cu") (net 4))
 (segment (start 125.15 33.85) (end 131 33.85) (width 0.4) (layer "F.Cu") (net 4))
 (segment (start 132.1275 36.45) (end 134.25 36.45) (width 0.4) (layer "F.Cu") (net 4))
 (segment (start 134.725 36.925) (end 134.725 37.45) (width 0.4) (layer "F.Cu") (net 4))
 (segment (start 124.1362 35.545) (end 124.1362 34.8638) (width 0.4) (layer "F.Cu") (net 4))
 (segment (start 131 33.85) (end 131.95 34.8) (width 0.4) (layer "F.Cu") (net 4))
 (segment (start 131.95 34.85) (end 132.1275 35.0275) (width 0.4) (layer "F.Cu") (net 4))
 (segment (start 134.25 36.45) (end 134.725 36.925) (width 0.4) (layer "F.Cu") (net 4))
 (segment (start 124.1362 34.8638) (end 125.15 33.85) (width 0.4) (layer "F.Cu") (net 4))
 (segment (start 131.95 34.8) (end 131.95 34.85) (width 0.4) (layer "F.Cu") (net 4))
 (segment (start 120.365 36.815) (end 124.1362 36.815) (width 0.4) (layer "F.Cu") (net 2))
 (segment (start 118.5 34.95) (end 120.365 36.815) (width 0.4) (layer "F.Cu") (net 2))
 (segment (start 117.1 34.95) (end 118.5 34.95) (width 0.4) (layer "F.Cu") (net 2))
 (segment (start 106.45 33.6) (end 106.45 30.05) (width 0.4) (layer "F.Cu") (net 5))
 (segment (start 106.45 36.6) (end 106.45 33.6) (width 0.4) (layer "F.Cu") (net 5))
 (segment (start 124.1362 38.085) (end 107.935 38.085) (width 0.4) (layer "F.Cu") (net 5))
 (segment (start 107.935 38.085) (end 106.45 36.6) (width 0.4) (layer "F.Cu") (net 5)))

